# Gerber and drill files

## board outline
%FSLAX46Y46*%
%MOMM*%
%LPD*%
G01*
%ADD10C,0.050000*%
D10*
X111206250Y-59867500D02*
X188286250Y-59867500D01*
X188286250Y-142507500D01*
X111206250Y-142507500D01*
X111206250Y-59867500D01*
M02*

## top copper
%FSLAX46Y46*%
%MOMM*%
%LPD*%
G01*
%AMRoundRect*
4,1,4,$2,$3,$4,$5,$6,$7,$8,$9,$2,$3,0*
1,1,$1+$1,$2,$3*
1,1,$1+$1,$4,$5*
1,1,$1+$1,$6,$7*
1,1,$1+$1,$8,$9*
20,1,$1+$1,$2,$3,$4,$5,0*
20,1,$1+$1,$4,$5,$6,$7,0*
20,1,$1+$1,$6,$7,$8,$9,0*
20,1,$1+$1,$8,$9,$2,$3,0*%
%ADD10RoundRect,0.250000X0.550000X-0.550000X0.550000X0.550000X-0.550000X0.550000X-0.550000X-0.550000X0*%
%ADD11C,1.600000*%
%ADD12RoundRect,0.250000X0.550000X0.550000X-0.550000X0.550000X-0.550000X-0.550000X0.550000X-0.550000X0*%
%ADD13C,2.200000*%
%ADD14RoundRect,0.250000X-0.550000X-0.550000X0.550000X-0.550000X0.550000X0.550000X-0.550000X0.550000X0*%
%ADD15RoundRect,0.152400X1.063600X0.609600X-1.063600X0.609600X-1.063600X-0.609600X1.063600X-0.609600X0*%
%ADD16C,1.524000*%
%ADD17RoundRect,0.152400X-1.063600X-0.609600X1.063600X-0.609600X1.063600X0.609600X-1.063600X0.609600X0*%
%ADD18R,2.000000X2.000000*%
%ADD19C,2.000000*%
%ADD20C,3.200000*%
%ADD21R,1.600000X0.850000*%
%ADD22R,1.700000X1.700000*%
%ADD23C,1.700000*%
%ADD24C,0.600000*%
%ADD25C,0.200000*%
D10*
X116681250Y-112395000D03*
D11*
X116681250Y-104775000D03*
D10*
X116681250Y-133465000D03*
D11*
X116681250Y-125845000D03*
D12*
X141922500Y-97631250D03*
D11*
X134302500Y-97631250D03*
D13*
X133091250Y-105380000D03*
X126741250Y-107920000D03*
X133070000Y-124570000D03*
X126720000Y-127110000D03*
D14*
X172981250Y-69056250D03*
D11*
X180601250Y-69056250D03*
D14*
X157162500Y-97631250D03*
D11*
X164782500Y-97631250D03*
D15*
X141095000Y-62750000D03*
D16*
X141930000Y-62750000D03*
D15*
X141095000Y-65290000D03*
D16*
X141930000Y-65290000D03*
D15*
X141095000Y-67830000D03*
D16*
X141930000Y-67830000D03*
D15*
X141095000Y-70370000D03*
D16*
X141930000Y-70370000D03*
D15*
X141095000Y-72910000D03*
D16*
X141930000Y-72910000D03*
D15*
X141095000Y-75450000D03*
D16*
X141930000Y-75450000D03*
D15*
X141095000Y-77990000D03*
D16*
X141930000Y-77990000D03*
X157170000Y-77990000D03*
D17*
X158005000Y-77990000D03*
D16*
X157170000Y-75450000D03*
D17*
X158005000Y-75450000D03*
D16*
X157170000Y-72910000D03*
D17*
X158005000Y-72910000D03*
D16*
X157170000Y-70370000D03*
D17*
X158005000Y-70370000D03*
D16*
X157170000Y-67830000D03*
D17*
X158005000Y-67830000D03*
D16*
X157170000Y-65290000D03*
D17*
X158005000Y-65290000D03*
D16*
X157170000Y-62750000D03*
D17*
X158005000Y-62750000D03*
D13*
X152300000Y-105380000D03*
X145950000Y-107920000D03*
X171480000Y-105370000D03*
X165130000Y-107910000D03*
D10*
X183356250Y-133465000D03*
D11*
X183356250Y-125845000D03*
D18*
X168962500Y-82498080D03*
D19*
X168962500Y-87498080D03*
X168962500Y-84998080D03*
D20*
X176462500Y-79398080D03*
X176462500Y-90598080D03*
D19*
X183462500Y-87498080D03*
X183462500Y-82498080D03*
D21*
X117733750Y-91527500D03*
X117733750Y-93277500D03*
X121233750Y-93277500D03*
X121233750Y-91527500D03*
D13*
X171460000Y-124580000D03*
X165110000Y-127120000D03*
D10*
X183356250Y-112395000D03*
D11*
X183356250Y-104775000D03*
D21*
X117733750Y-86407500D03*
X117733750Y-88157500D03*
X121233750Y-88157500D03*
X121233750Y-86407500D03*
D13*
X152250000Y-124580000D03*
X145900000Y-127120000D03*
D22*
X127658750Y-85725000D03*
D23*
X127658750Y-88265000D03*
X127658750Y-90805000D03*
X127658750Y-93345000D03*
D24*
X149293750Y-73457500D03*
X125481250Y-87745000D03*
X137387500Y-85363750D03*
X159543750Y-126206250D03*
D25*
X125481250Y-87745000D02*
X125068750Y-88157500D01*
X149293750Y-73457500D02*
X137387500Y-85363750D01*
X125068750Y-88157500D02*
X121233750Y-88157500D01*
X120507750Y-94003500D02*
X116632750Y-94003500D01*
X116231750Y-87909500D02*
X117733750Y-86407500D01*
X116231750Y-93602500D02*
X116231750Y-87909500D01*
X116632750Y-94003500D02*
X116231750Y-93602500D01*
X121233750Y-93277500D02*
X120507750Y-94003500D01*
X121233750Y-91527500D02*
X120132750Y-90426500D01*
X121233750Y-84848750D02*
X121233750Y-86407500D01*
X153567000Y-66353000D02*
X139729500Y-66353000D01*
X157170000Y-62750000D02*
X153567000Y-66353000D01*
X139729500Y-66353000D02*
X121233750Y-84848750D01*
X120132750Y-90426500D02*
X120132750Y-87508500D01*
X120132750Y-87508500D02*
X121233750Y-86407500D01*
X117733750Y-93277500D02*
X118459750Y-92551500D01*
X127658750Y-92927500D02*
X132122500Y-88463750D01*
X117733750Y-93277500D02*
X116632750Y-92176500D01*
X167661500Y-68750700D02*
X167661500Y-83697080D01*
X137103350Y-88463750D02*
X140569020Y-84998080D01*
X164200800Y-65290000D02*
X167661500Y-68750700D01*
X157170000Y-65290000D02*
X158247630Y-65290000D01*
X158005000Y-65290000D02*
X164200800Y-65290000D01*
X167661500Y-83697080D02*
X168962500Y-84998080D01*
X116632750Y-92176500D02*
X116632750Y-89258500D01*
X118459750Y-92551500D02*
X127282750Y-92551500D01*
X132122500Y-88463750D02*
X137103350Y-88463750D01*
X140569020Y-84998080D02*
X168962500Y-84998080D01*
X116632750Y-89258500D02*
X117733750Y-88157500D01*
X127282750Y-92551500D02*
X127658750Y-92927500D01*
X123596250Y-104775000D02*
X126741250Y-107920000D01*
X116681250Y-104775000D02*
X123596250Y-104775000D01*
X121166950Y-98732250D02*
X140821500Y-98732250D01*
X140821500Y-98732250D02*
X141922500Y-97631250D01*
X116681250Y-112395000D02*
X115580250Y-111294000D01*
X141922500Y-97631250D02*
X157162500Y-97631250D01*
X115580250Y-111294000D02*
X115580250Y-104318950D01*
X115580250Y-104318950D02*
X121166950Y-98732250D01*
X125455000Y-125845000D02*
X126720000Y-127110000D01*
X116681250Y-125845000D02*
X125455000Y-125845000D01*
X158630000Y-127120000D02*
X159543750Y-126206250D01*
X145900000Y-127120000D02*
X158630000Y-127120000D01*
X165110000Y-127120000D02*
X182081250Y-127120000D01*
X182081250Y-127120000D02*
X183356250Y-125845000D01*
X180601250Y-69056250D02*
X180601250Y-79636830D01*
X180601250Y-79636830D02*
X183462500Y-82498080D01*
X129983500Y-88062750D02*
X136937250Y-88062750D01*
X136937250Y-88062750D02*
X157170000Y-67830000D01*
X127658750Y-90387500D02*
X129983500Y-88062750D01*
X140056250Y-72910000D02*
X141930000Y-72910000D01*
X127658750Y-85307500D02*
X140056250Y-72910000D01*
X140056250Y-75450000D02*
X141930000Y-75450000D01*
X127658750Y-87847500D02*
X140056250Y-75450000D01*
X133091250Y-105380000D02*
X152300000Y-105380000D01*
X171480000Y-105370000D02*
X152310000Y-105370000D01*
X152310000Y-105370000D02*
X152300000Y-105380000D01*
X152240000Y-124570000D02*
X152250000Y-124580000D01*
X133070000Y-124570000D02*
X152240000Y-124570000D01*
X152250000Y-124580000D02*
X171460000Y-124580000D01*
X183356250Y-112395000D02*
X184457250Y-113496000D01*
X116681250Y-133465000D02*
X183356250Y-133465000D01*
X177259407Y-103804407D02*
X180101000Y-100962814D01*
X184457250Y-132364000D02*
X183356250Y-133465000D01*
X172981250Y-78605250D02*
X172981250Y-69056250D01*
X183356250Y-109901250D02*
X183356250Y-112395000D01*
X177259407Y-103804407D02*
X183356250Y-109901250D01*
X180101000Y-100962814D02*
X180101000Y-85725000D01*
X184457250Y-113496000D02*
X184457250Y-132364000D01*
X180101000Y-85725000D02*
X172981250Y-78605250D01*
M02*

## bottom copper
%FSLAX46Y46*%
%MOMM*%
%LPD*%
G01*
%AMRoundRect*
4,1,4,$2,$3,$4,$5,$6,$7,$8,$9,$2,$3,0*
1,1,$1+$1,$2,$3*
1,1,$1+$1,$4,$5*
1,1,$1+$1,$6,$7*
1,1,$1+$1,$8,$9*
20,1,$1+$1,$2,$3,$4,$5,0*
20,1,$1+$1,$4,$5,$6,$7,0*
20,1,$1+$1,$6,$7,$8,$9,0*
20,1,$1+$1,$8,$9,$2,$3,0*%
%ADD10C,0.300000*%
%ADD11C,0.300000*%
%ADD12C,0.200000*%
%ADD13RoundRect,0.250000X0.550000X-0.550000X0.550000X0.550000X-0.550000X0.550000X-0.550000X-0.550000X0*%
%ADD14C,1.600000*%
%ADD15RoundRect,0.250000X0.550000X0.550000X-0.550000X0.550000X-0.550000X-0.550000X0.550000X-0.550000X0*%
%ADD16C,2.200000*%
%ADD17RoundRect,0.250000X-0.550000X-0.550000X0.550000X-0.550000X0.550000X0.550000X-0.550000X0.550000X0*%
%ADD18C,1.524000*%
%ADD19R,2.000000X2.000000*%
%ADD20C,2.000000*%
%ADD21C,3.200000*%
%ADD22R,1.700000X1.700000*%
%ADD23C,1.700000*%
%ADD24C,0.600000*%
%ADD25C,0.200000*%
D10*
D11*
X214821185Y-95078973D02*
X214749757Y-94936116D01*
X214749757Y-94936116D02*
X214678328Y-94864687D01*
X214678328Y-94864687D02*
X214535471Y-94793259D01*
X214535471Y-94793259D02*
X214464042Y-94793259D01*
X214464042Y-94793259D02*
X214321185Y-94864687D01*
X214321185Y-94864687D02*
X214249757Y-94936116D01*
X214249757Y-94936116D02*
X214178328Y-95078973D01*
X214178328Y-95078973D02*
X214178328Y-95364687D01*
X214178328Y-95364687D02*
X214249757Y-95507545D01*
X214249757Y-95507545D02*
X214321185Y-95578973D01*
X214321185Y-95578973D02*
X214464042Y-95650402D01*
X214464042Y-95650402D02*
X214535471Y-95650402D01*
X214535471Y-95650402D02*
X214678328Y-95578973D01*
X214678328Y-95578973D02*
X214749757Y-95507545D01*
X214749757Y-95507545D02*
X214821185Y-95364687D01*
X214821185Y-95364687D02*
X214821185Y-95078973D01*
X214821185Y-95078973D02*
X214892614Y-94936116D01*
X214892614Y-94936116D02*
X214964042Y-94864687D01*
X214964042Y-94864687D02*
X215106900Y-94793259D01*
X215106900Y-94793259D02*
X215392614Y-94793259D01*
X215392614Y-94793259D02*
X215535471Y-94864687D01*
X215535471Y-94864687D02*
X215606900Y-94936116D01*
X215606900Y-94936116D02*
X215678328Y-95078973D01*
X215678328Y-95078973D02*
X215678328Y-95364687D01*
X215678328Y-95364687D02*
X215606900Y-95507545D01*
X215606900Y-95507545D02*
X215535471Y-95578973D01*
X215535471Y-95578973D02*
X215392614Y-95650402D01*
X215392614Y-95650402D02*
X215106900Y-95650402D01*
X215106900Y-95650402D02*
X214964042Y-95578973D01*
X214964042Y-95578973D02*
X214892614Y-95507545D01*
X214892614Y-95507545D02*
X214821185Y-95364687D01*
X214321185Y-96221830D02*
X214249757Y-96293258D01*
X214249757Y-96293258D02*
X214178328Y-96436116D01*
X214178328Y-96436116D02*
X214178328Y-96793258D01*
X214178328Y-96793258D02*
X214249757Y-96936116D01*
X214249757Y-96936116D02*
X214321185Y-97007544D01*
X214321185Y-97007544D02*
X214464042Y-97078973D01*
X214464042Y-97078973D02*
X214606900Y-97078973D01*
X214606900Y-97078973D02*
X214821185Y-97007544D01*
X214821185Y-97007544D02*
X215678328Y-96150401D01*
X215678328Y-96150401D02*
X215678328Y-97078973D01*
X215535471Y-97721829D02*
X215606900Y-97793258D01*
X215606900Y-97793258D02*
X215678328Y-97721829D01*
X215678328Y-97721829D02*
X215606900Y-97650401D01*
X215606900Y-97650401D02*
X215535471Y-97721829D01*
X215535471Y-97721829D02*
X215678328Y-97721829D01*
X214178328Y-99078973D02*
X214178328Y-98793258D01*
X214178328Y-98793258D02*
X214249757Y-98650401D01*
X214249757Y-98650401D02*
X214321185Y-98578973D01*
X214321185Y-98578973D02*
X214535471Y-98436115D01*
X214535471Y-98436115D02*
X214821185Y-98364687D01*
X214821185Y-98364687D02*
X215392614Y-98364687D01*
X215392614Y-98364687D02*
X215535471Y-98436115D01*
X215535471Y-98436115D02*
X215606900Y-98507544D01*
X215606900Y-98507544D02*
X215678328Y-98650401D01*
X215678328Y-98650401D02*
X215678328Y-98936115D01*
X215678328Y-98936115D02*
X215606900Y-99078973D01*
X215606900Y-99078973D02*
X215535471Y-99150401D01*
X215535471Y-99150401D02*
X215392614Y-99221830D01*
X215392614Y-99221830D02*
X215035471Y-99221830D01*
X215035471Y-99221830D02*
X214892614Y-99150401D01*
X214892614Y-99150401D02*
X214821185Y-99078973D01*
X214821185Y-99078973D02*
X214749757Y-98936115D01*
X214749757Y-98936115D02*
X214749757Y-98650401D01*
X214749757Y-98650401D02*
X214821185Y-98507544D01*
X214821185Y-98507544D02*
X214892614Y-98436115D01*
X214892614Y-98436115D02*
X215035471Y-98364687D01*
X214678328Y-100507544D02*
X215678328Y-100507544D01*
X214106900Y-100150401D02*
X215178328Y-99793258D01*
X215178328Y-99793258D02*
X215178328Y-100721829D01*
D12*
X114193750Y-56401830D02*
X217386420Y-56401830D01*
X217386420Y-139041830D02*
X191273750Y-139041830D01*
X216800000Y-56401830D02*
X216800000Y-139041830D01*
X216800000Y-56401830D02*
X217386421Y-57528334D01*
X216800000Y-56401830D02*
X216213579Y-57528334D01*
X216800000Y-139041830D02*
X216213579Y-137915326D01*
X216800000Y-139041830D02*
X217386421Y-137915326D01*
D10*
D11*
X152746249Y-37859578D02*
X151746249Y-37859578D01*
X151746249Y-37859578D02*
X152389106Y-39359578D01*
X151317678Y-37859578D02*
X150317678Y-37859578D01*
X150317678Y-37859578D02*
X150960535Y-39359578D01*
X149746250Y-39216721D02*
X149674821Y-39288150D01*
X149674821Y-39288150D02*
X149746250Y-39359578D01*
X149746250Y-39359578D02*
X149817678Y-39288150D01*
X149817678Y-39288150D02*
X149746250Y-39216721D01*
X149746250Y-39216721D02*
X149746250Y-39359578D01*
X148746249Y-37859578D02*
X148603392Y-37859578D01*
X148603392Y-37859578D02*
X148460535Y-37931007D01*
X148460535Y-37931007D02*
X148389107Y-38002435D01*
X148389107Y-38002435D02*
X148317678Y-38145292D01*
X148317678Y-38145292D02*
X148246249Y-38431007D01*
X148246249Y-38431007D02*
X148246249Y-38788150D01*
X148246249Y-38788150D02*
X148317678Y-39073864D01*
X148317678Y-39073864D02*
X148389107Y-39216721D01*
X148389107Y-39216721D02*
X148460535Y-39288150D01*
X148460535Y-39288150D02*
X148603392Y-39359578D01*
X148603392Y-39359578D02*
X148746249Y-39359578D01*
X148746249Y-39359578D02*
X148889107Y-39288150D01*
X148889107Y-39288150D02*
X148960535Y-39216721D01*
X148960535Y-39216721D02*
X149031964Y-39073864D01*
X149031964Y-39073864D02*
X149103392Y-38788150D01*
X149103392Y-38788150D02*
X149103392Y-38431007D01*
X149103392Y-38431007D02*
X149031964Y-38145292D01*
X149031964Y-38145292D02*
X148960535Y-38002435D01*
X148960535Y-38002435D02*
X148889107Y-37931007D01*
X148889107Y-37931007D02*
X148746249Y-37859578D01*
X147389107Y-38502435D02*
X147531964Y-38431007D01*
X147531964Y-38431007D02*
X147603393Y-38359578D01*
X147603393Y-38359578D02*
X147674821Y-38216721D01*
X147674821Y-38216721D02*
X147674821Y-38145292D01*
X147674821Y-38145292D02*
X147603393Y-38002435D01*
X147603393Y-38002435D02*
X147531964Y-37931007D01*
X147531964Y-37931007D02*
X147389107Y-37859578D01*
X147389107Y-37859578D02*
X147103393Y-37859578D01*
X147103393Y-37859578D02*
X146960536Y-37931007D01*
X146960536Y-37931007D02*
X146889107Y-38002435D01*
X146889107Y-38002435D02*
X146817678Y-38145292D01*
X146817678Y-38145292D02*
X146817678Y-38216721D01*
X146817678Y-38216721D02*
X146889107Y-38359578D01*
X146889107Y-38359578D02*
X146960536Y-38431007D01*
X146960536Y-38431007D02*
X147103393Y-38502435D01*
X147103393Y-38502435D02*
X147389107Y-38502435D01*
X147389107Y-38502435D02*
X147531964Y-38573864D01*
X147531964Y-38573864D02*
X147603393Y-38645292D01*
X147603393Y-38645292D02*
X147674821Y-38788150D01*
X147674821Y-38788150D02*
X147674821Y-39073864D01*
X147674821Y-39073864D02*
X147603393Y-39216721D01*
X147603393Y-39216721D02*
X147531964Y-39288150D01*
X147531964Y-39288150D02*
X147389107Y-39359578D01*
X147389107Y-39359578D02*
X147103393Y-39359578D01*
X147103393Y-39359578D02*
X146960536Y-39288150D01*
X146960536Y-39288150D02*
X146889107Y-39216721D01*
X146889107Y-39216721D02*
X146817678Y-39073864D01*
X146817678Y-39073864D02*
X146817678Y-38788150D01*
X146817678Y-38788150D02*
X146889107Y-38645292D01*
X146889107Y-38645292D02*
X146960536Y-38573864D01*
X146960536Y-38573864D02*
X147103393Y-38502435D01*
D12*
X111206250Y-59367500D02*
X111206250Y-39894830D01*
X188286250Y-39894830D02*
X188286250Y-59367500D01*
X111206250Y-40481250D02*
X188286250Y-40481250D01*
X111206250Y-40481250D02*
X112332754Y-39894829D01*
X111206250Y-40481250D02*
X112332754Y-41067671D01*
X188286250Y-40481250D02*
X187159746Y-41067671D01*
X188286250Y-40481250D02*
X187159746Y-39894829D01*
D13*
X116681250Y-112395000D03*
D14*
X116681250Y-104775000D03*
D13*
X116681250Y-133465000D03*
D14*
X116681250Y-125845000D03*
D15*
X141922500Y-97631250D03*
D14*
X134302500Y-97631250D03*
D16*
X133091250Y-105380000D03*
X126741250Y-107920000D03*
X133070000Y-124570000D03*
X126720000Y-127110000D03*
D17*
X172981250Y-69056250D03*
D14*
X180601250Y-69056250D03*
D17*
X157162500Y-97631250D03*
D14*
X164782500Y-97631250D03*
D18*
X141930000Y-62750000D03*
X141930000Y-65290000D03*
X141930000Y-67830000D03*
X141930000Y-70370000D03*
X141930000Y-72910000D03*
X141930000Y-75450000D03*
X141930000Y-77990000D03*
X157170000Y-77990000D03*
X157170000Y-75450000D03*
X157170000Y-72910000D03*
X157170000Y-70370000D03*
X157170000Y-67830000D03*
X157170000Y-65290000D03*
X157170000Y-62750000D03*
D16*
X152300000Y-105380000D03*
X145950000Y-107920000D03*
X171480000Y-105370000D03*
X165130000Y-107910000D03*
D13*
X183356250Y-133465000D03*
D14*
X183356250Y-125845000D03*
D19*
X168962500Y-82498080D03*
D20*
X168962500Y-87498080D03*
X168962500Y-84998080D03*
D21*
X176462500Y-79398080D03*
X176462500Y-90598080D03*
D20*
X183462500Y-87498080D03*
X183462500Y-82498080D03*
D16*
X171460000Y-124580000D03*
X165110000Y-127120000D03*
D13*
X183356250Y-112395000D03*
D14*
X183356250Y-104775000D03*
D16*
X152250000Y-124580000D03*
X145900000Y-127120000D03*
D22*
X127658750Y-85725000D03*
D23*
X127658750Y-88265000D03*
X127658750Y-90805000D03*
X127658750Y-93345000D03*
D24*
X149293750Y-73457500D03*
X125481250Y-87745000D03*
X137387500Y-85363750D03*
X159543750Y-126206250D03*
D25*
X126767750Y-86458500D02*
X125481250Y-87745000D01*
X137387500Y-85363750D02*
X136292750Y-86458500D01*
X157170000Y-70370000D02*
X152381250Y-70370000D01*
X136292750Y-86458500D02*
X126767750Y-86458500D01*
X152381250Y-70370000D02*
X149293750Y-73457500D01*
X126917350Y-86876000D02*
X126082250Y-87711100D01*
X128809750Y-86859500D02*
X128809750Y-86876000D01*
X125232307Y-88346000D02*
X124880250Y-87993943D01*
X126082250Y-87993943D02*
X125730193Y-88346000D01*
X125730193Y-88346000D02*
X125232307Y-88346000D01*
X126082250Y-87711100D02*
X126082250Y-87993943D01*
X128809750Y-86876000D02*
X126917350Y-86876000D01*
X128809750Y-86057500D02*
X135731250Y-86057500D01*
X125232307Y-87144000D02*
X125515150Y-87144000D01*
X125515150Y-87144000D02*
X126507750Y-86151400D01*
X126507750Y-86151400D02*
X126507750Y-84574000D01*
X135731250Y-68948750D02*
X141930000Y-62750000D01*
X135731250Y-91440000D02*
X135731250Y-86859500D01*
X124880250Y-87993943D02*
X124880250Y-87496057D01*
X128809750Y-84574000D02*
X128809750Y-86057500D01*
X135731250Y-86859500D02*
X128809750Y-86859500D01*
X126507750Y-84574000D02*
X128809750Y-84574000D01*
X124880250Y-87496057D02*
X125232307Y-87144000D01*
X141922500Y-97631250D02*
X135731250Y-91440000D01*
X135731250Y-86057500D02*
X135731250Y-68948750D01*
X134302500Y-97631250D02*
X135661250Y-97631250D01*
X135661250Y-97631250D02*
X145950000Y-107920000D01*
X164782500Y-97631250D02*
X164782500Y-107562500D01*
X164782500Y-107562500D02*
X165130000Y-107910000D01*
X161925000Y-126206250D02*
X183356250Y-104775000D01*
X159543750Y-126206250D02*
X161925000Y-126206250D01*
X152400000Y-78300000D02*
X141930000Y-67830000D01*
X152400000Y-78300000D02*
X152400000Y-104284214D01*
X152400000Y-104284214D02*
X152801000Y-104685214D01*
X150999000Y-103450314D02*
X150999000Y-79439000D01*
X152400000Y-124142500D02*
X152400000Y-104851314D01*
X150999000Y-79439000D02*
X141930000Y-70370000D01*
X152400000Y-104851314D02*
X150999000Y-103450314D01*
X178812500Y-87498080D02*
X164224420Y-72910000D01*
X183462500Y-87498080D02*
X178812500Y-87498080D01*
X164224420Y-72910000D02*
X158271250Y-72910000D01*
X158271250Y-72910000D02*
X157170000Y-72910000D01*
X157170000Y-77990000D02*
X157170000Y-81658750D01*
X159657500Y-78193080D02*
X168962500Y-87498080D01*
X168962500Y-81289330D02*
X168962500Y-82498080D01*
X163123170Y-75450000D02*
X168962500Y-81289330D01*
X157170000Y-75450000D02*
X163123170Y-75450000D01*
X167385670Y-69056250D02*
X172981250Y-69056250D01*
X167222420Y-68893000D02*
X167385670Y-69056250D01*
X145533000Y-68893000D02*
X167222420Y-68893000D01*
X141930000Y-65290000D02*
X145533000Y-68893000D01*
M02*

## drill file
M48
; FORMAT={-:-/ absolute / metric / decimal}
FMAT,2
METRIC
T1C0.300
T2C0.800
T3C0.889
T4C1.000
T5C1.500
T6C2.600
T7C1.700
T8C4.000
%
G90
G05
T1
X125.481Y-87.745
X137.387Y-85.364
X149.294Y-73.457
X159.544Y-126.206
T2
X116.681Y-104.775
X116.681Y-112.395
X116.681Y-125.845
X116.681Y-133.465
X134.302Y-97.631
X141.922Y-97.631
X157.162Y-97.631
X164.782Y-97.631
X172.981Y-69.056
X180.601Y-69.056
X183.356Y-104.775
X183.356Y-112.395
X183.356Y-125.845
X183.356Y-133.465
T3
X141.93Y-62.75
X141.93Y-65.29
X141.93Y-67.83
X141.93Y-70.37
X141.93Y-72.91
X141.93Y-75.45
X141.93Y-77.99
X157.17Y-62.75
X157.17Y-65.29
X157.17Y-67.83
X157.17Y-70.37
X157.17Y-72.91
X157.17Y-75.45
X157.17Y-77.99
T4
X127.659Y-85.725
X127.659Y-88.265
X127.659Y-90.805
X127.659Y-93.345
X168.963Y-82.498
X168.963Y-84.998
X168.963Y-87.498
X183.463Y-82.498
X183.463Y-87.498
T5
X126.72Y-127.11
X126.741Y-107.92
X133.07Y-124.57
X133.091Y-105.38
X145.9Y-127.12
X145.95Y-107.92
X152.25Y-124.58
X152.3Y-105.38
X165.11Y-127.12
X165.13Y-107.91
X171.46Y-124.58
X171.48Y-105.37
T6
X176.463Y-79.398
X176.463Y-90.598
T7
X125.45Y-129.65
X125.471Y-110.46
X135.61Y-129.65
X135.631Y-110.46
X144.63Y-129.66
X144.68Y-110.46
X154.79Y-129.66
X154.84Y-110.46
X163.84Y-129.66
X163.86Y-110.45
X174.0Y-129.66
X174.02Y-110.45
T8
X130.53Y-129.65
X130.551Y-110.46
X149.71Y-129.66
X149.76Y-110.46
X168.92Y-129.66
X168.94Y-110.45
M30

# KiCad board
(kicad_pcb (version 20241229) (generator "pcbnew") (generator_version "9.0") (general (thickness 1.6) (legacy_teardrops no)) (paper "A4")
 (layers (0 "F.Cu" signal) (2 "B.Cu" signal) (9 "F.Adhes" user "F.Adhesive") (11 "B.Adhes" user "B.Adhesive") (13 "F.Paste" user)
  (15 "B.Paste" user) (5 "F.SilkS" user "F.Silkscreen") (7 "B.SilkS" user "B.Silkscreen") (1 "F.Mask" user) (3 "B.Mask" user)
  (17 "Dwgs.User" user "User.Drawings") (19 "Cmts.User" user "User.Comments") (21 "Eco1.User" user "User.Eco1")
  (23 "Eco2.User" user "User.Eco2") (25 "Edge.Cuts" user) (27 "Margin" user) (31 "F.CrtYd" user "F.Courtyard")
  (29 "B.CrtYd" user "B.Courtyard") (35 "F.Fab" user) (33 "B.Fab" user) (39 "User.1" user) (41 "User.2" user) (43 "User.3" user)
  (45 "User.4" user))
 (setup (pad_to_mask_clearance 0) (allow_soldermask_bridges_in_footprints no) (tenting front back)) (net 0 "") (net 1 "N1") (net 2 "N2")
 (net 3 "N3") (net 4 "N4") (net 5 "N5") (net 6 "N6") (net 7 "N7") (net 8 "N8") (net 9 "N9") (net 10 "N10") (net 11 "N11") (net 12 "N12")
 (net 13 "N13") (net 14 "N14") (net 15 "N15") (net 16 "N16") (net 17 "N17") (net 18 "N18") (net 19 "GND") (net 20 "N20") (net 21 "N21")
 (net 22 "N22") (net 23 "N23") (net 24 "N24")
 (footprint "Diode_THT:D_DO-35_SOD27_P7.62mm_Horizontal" (layer "F.Cu") (at 116.68125 112.395 90)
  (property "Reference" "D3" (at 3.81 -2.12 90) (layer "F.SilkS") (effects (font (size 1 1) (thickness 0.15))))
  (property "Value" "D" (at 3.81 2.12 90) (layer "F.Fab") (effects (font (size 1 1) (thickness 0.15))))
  (pad "1" thru_hole roundrect (at 0 0 90) (size 1.6 1.6) (drill 0.8) (layers "*.Cu" "*.Mask") (remove_unused_layers no)
   (roundrect_rratio 0.15625) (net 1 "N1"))
  (pad "2" thru_hole circle (at 7.62 0 90) (size 1.6 1.6) (drill 0.8) (layers "*.Cu" "*.Mask") (remove_unused_layers no) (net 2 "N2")))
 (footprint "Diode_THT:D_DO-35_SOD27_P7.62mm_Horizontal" (layer "F.Cu") (at 116.68125 133.465 90)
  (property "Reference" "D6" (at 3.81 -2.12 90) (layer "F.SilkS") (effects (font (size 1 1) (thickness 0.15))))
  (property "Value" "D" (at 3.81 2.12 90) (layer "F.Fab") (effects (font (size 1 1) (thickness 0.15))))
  (pad "1" thru_hole roundrect (at 0 0 90) (size 1.6 1.6) (drill 0.8) (layers "*.Cu" "*.Mask") (remove_unused_layers no)
   (roundrect_rratio 0.15625) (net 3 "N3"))
  (pad "2" thru_hole circle (at 7.62 0 90) (size 1.6 1.6) (drill 0.8) (layers "*.Cu" "*.Mask") (remove_unused_layers no) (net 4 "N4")))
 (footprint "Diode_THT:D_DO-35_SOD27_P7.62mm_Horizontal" (layer "F.Cu") (at 141.9225 97.63125 180)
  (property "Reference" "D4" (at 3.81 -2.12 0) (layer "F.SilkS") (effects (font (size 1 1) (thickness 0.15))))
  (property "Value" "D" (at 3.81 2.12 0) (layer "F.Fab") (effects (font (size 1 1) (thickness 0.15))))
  (pad "1" thru_hole roundrect (at 0 0 180) (size 1.6 1.6) (drill 0.8) (layers "*.Cu" "*.Mask") (remove_unused_layers no)
   (roundrect_rratio 0.15625) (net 1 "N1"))
  (pad "2" thru_hole circle (at 7.62 0 180) (size 1.6 1.6) (drill 0.8) (layers "*.Cu" "*.Mask") (remove_unused_layers no) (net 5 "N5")))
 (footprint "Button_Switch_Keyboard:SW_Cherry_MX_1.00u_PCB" (layer "F.Cu") (at 133.09125 105.38)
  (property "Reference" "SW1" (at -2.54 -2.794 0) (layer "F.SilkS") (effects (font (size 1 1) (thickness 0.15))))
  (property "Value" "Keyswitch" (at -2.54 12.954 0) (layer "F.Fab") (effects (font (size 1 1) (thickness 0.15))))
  (pad "" np_thru_hole circle (at -7.62 5.08) (size 1.7 1.7) (drill 1.7) (layers "*.Cu" "*.Mask"))
  (pad "" np_thru_hole circle (at -2.54 5.08) (size 4 4) (drill 4) (layers "*.Cu" "*.Mask"))
  (pad "" np_thru_hole circle (at 2.54 5.08) (size 1.7 1.7) (drill 1.7) (layers "*.Cu" "*.Mask"))
  (pad "1" thru_hole circle (at 0 0) (size 2.2 2.2) (drill 1.5) (layers "*.Cu" "*.Mask") (remove_unused_layers no) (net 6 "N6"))
  (pad "2" thru_hole circle (at -6.35 2.54) (size 2.2 2.2) (drill 1.5) (layers "*.Cu" "*.Mask") (remove_unused_layers no) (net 2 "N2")))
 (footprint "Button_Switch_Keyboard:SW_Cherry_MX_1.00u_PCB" (layer "F.Cu") (at 133.07 124.57)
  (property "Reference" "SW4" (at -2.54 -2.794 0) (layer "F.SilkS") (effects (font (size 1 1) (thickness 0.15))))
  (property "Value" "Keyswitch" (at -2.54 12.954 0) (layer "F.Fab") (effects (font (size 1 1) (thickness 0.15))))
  (pad "" np_thru_hole circle (at -7.62 5.08) (size 1.7 1.7) (drill 1.7) (layers "*.Cu" "*.Mask"))
  (pad "" np_thru_hole circle (at -2.54 5.08) (size 4 4) (drill 4) (layers "*.Cu" "*.Mask"))
  (pad "" np_thru_hole circle (at 2.54 5.08) (size 1.7 1.7) (drill 1.7) (layers "*.Cu" "*.Mask"))
  (pad "1" thru_hole circle (at 0 0) (size 2.2 2.2) (drill 1.5) (layers "*.Cu" "*.Mask") (remove_unused_layers no) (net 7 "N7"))
  (pad "2" thru_hole circle (at -6.35 2.54) (size 2.2 2.2) (drill 1.5) (layers "*.Cu" "*.Mask") (remove_unused_layers no) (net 4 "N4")))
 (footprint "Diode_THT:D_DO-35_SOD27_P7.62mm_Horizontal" (layer "F.Cu") (at 172.98125 69.05625)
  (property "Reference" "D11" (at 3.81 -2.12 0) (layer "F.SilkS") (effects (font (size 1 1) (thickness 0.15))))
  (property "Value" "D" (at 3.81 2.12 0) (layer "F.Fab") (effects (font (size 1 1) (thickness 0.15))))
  (pad "1" thru_hole roundrect (at 0 0) (size 1.6 1.6) (drill 0.8) (layers "*.Cu" "*.Mask") (remove_unused_layers no)
   (roundrect_rratio 0.15625) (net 3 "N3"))
  (pad "2" thru_hole circle (at 7.62 0) (size 1.6 1.6) (drill 0.8) (layers "*.Cu" "*.Mask") (remove_unused_layers no) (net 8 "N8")))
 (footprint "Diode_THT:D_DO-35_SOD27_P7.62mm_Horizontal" (layer "F.Cu") (at 157.1625 97.63125)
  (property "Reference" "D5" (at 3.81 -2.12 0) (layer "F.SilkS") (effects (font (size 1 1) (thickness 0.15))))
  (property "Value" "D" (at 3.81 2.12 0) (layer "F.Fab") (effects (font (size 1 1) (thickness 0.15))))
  (pad "1" thru_hole roundrect (at 0 0) (size 1.6 1.6) (drill 0.8) (layers "*.Cu" "*.Mask") (remove_unused_layers no)
   (roundrect_rratio 0.15625) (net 1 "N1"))
  (pad "2" thru_hole circle (at 7.62 0) (size 1.6 1.6) (drill 0.8) (layers "*.Cu" "*.Mask") (remove_unused_layers no) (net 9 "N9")))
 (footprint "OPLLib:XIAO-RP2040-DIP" (layer "F.Cu") (at 149.55 70.37)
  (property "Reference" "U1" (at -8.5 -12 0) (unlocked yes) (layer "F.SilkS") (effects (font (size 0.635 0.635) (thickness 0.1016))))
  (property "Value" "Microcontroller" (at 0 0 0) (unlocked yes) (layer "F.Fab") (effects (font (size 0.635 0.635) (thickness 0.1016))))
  (pad "1" smd roundrect (at -8.455 -7.62 180) (size 2.432 1.524) (layers "F.Cu" "F.Mask") (roundrect_rratio 0.1) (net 1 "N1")
   (thermal_bridge_angle 45))
  (pad "1" thru_hole circle (at -7.62 -7.62 180) (size 1.524 1.524) (drill 0.889) (layers "*.Cu" "*.Mask") (remove_unused_layers no)
   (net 1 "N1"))
  (pad "2" smd roundrect (at -8.455 -5.08 180) (size 2.432 1.524) (layers "F.Cu" "F.Mask") (roundrect_rratio 0.1) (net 3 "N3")
   (thermal_bridge_angle 45))
  (pad "2" thru_hole circle (at -7.62 -5.08 180) (size 1.524 1.524) (drill 0.889) (layers "*.Cu" "*.Mask") (remove_unused_layers no)
   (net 3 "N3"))
  (pad "3" smd roundrect (at -8.455 -2.54 180) (size 2.432 1.524) (layers "F.Cu" "F.Mask") (roundrect_rratio 0.1) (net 6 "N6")
   (thermal_bridge_angle 45))
  (pad "3" thru_hole circle (at -7.62 -2.54 180) (size 1.524 1.524) (drill 0.889) (layers "*.Cu" "*.Mask") (remove_unused_layers no)
   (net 6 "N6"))
  (pad "4" smd roundrect (at -8.455 0 180) (size 2.432 1.524) (layers "F.Cu" "F.Mask") (roundrect_rratio 0.1) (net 7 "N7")
   (thermal_bridge_angle 45))
  (pad "4" thru_hole circle (at -7.62 0 180) (size 1.524 1.524) (drill 0.889) (layers "*.Cu" "*.Mask") (remove_unused_layers no)
   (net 7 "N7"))
  (pad "5" smd roundrect (at -8.455 2.54 180) (size 2.432 1.524) (layers "F.Cu" "F.Mask") (roundrect_rratio 0.1) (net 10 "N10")
   (thermal_bridge_angle 45))
  (pad "5" thru_hole circle (at -7.62 2.54 180) (size 1.524 1.524) (drill 0.889) (layers "*.Cu" "*.Mask") (remove_unused_layers no)
   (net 10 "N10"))
  (pad "6" smd roundrect (at -8.455 5.08 180) (size 2.432 1.524) (layers "F.Cu" "F.Mask") (roundrect_rratio 0.1) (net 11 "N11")
   (thermal_bridge_angle 45))
  (pad "6" thru_hole circle (at -7.62 5.08 180) (size 1.524 1.524) (drill 0.889) (layers "*.Cu" "*.Mask") (remove_unused_layers no)
   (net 11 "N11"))
  (pad "7" smd roundrect (at -8.455 7.62 180) (size 2.432 1.524) (layers "F.Cu" "F.Mask") (roundrect_rratio 0.1) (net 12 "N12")
   (thermal_bridge_angle 45))
  (pad "7" thru_hole circle (at -7.62 7.62 180) (size 1.524 1.524) (drill 0.889) (layers "*.Cu" "*.Mask") (remove_unused_layers no)
   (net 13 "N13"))
  (pad "8" thru_hole circle (at 7.62 7.62) (size 1.524 1.524) (drill 0.889) (layers "*.Cu" "*.Mask") (remove_unused_layers no)
   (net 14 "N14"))
  (pad "8" smd roundrect (at 8.455 7.62) (size 2.432 1.524) (layers "F.Cu" "F.Mask") (roundrect_rratio 0.1) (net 14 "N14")
   (thermal_bridge_angle 45))
  (pad "9" thru_hole circle (at 7.62 5.08) (size 1.524 1.524) (drill 0.889) (layers "*.Cu" "*.Mask") (remove_unused_layers no)
   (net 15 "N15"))
  (pad "9" smd roundrect (at 8.455 5.08) (size 2.432 1.524) (layers "F.Cu" "F.Mask") (roundrect_rratio 0.1) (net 15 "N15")
   (thermal_bridge_angle 45))
  (pad "10" thru_hole circle (at 7.62 2.54) (size 1.524 1.524) (drill 0.889) (layers "*.Cu" "*.Mask") (remove_unused_layers no)
   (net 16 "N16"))
  (pad "10" smd roundrect (at 8.455 2.54) (size 2.432 1.524) (layers "F.Cu" "F.Mask") (roundrect_rratio 0.1) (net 16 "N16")
   (thermal_bridge_angle 45))
  (pad "11" thru_hole circle (at 7.62 0) (size 1.524 1.524) (drill 0.889) (layers "*.Cu" "*.Mask") (remove_unused_layers no) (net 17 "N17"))
  (pad "11" smd roundrect (at 8.455 0) (size 2.432 1.524) (layers "F.Cu" "F.Mask") (roundrect_rratio 0.1) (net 17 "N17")
   (thermal_bridge_angle 45))
  (pad "12" thru_hole circle (at 7.62 -2.54) (size 1.524 1.524) (drill 0.889) (layers "*.Cu" "*.Mask") (remove_unused_layers no)
   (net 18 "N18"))
  (pad "12" smd roundrect (at 8.455 -2.54) (size 2.432 1.524) (layers "F.Cu" "F.Mask") (roundrect_rratio 0.1) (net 18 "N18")
   (thermal_bridge_angle 45))
  (pad "13" thru_hole circle (at 7.62 -5.08) (size 1.524 1.524) (drill 0.889) (layers "*.Cu" "*.Mask") (remove_unused_layers no)
   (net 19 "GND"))
  (pad "13" smd roundrect (at 8.455 -5.08) (size 2.432 1.524) (layers "F.Cu" "F.Mask") (roundrect_rratio 0.1) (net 19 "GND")
   (thermal_bridge_angle 45))
  (pad "14" thru_hole circle (at 7.62 -7.62) (size 1.524 1.524) (drill 0.889) (layers "*.Cu" "*.Mask") (remove_unused_layers no)
   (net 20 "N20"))
  (pad "14" smd roundrect (at 8.455 -7.62) (size 2.432 1.524) (layers "F.Cu" "F.Mask") (roundrect_rratio 0.1) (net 20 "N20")
   (thermal_bridge_angle 45)))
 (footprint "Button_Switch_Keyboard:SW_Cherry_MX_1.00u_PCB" (layer "F.Cu") (at 152.3 105.38)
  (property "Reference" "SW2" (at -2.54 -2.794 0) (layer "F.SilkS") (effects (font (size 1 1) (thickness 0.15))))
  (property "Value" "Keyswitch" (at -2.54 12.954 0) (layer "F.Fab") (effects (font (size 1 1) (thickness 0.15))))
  (pad "" np_thru_hole circle (at -7.62 5.08) (size 1.7 1.7) (drill 1.7) (layers "*.Cu" "*.Mask"))
  (pad "" np_thru_hole circle (at -2.54 5.08) (size 4 4) (drill 4) (layers "*.Cu" "*.Mask"))
  (pad "" np_thru_hole circle (at 2.54 5.08) (size 1.7 1.7) (drill 1.7) (layers "*.Cu" "*.Mask"))
  (pad "1" thru_hole circle (at 0 0) (size 2.2 2.2) (drill 1.5) (layers "*.Cu" "*.Mask") (remove_unused_layers no) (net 6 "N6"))
  (pad "2" thru_hole circle (at -6.35 2.54) (size 2.2 2.2) (drill 1.5) (layers "*.Cu" "*.Mask") (remove_unused_layers no) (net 5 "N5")))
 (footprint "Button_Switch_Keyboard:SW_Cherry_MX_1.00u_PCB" (layer "F.Cu") (at 171.48 105.37)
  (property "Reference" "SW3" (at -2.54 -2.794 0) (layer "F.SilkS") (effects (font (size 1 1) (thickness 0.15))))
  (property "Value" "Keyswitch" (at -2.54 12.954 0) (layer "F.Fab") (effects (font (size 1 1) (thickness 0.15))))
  (pad "" np_thru_hole circle (at -7.62 5.08) (size 1.7 1.7) (drill 1.7) (layers "*.Cu" "*.Mask"))
  (pad "" np_thru_hole circle (at -2.54 5.08) (size 4 4) (drill 4) (layers "*.Cu" "*.Mask"))
  (pad "" np_thru_hole circle (at 2.54 5.08) (size 1.7 1.7) (drill 1.7) (layers "*.Cu" "*.Mask"))
  (pad "1" thru_hole circle (at 0 0) (size 2.2 2.2) (drill 1.5) (layers "*.Cu" "*.Mask") (remove_unused_layers no) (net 6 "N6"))
  (pad "2" thru_hole circle (at -6.35 2.54) (size 2.2 2.2) (drill 1.5) (layers "*.Cu" "*.Mask") (remove_unused_layers no) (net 9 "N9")))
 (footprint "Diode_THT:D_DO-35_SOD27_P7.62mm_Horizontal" (layer "F.Cu") (at 183.35625 133.465 90)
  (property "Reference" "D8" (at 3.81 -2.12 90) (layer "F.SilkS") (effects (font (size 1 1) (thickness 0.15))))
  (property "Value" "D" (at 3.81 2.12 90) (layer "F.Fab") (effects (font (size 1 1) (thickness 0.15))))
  (pad "1" thru_hole roundrect (at 0 0 90) (size 1.6 1.6) (drill 0.8) (layers "*.Cu" "*.Mask") (remove_unused_layers no)
   (roundrect_rratio 0.15625) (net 3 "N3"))
  (pad "2" thru_hole circle (at 7.62 0 90) (size 1.6 1.6) (drill 0.8) (layers "*.Cu" "*.Mask") (remove_unused_layers no) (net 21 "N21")))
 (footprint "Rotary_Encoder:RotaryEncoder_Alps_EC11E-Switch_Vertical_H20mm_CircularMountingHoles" (layer "F.Cu") (at 168.9625 82.49808)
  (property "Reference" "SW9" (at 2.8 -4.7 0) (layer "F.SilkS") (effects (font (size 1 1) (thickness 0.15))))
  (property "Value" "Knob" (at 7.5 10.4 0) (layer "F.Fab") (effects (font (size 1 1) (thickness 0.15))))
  (pad "A" thru_hole rect (at 0 0) (size 2 2) (drill 1) (layers "*.Cu" "*.Mask") (remove_unused_layers no) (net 15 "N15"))
  (pad "B" thru_hole circle (at 0 5) (size 2 2) (drill 1) (layers "*.Cu" "*.Mask") (remove_unused_layers no) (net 14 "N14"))
  (pad "C" thru_hole circle (at 0 2.5) (size 2 2) (drill 1) (layers "*.Cu" "*.Mask") (remove_unused_layers no) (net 19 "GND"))
  (pad "MP" thru_hole circle (at 7.5 -3.1) (size 3.2 3.2) (drill 2.6) (layers "*.Cu" "*.Mask") (remove_unused_layers no))
  (pad "MP" thru_hole circle (at 7.5 8.1) (size 3.2 3.2) (drill 2.6) (layers "*.Cu" "*.Mask") (remove_unused_layers no))
  (pad "S1" thru_hole circle (at 14.5 5) (size 2 2) (drill 1) (layers "*.Cu" "*.Mask") (remove_unused_layers no) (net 16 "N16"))
  (pad "S2" thru_hole circle (at 14.5 0) (size 2 2) (drill 1) (layers "*.Cu" "*.Mask") (remove_unused_layers no) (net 8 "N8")))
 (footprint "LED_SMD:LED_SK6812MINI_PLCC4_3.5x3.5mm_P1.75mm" (layer "F.Cu") (at 119.48375 92.4025)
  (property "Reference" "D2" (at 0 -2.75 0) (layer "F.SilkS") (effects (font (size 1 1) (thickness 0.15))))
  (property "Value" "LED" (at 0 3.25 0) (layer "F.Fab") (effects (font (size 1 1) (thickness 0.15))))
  (pad "1" smd rect (at -1.75 -0.875) (size 1.6 0.85) (layers "F.Cu" "F.Mask" "F.Paste") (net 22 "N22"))
  (pad "2" smd rect (at -1.75 0.875) (size 1.6 0.85) (layers "F.Cu" "F.Mask" "F.Paste") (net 19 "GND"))
  (pad "3" smd rect (at 1.75 0.875) (size 1.6 0.85) (layers "F.Cu" "F.Mask" "F.Paste") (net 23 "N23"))
  (pad "4" smd rect (at 1.75 -0.875) (size 1.6 0.85) (layers "F.Cu" "F.Mask" "F.Paste") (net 20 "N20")))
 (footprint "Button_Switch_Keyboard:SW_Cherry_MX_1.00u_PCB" (layer "F.Cu") (at 171.46 124.58)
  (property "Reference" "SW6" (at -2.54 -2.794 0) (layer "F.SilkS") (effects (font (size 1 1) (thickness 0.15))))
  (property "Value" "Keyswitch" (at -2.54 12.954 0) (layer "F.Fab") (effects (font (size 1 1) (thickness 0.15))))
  (pad "" np_thru_hole circle (at -7.62 5.08) (size 1.7 1.7) (drill 1.7) (layers "*.Cu" "*.Mask"))
  (pad "" np_thru_hole circle (at -2.54 5.08) (size 4 4) (drill 4) (layers "*.Cu" "*.Mask"))
  (pad "" np_thru_hole circle (at 2.54 5.08) (size 1.7 1.7) (drill 1.7) (layers "*.Cu" "*.Mask"))
  (pad "1" thru_hole circle (at 0 0) (size 2.2 2.2) (drill 1.5) (layers "*.Cu" "*.Mask") (remove_unused_layers no) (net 7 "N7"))
  (pad "2" thru_hole circle (at -6.35 2.54) (size 2.2 2.2) (drill 1.5) (layers "*.Cu" "*.Mask") (remove_unused_layers no) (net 21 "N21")))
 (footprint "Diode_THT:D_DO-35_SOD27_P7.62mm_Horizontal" (layer "F.Cu") (at 183.35625 112.395 90)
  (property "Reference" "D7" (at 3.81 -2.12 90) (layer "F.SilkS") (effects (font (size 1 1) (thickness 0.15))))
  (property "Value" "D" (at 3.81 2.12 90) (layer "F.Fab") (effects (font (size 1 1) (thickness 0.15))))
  (pad "1" thru_hole roundrect (at 0 0 90) (size 1.6 1.6) (drill 0.8) (layers "*.Cu" "*.Mask") (remove_unused_layers no)
   (roundrect_rratio 0.15625) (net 3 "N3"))
  (pad "2" thru_hole circle (at 7.62 0 90) (size 1.6 1.6) (drill 0.8) (layers "*.Cu" "*.Mask") (remove_unused_layers no) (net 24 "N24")))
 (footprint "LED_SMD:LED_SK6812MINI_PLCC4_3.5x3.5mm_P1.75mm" (layer "F.Cu") (at 119.48375 87.2825)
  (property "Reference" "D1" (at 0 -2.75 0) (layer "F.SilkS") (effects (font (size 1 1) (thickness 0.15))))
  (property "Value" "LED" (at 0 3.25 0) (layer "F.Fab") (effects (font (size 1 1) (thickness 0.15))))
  (pad "1" smd rect (at -1.75 -0.875) (size 1.6 0.85) (layers "F.Cu" "F.Mask" "F.Paste") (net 23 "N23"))
  (pad "2" smd rect (at -1.75 0.875) (size 1.6 0.85) (layers "F.Cu" "F.Mask" "F.Paste") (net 19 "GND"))
  (pad "3" smd rect (at 1.75 0.875) (size 1.6 0.85) (layers "F.Cu" "F.Mask" "F.Paste") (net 17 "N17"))
  (pad "4" smd rect (at 1.75 -0.875) (size 1.6 0.85) (layers "F.Cu" "F.Mask" "F.Paste") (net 20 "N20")))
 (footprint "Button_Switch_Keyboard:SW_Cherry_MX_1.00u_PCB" (layer "F.Cu") (at 152.25 124.58)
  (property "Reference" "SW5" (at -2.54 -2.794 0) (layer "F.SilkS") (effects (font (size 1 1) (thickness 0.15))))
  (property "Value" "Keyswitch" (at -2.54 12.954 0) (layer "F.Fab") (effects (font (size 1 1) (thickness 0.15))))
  (pad "" np_thru_hole circle (at -7.62 5.08) (size 1.7 1.7) (drill 1.7) (layers "*.Cu" "*.Mask"))
  (pad "" np_thru_hole circle (at -2.54 5.08) (size 4 4) (drill 4) (layers "*.Cu" "*.Mask"))
  (pad "" np_thru_hole circle (at 2.54 5.08) (size 1.7 1.7) (drill 1.7) (layers "*.Cu" "*.Mask"))
  (pad "1" thru_hole circle (at 0 0) (size 2.2 2.2) (drill 1.5) (layers "*.Cu" "*.Mask") (remove_unused_layers no) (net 7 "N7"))
  (pad "2" thru_hole circle (at -6.35 2.54) (size 2.2 2.2) (drill 1.5) (layers "*.Cu" "*.Mask") (remove_unused_layers no) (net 24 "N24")))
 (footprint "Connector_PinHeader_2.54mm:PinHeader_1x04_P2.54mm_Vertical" (layer "F.Cu") (at 127.65875 85.725)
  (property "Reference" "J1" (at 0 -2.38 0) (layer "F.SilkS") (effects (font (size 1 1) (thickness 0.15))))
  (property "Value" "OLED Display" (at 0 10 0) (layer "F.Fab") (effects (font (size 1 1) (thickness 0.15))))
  (pad "1" thru_hole rect (at 0 0) (size 1.7 1.7) (drill 1) (layers "*.Cu" "*.Mask") (remove_unused_layers no) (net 10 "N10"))
  (pad "2" thru_hole circle (at 0 2.54) (size 1.7 1.7) (drill 1) (layers "*.Cu" "*.Mask") (remove_unused_layers no) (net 11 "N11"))
  (pad "3" thru_hole circle (at 0 5.08) (size 1.7 1.7) (drill 1) (layers "*.Cu" "*.Mask") (remove_unused_layers no) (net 18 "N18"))
  (pad "4" thru_hole circle (at 0 7.62) (size 1.7 1.7) (drill 1) (layers "*.Cu" "*.Mask") (remove_unused_layers no) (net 19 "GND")))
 (gr_rect (start 111.20625 59.8675) (end 188.28625 142.5075) (stroke (width 0.05) (type solid)) (fill no) (layer "Edge.Cuts"))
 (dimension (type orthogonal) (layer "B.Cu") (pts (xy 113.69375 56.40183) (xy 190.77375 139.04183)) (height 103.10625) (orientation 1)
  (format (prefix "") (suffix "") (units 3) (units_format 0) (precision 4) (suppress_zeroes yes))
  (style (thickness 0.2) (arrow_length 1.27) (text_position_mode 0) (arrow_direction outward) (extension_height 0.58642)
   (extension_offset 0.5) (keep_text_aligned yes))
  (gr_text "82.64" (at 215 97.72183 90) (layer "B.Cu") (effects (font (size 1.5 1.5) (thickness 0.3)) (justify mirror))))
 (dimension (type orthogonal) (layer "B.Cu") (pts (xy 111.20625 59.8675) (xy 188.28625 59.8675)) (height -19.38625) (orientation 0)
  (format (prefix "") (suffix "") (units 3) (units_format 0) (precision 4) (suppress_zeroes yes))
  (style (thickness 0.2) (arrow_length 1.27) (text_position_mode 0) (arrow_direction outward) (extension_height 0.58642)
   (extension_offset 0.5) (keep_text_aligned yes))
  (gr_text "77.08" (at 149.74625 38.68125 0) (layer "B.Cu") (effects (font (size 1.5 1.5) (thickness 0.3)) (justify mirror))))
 (segment (start 125.48125 87.745) (end 125.06875 88.1575) (width 0.2) (layer "F.Cu") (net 17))
 (segment (start 149.29375 73.4575) (end 137.3875 85.36375) (width 0.2) (layer "F.Cu") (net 17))
 (segment (start 125.06875 88.1575) (end 121.23375 88.1575) (width 0.2) (layer "F.Cu") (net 17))
 (via (at 149.29375 73.4575) (size 0.6) (drill 0.3) (layers "F.Cu" "B.Cu") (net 17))
 (via (at 125.48125 87.745) (size 0.6) (drill 0.3) (layers "F.Cu" "B.Cu") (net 17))
 (via (at 137.3875 85.36375) (size 0.6) (drill 0.3) (layers "F.Cu" "B.Cu") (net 17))
 (segment (start 126.76775 86.4585) (end 125.48125 87.745) (width 0.2) (layer "B.Cu") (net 17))
 (segment (start 137.3875 85.36375) (end 136.29275 86.4585) (width 0.2) (layer "B.Cu") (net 17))
 (segment (start 157.17 70.37) (end 152.38125 70.37) (width 0.2) (layer "B.Cu") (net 17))
 (segment (start 136.29275 86.4585) (end 126.76775 86.4585) (width 0.2) (layer "B.Cu") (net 17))
 (segment (start 152.38125 70.37) (end 149.29375 73.4575) (width 0.2) (layer "B.Cu") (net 17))
 (segment (start 120.50775 94.0035) (end 116.63275 94.0035) (width 0.2) (layer "F.Cu") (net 23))
 (segment (start 116.23175 87.9095) (end 117.73375 86.4075) (width 0.2) (layer "F.Cu") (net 23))
 (segment (start 116.23175 93.6025) (end 116.23175 87.9095) (width 0.2) (layer "F.Cu") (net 23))
 (segment (start 116.63275 94.0035) (end 116.23175 93.6025) (width 0.2) (layer "F.Cu") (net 23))
 (segment (start 121.23375 93.2775) (end 120.50775 94.0035) (width 0.2) (layer "F.Cu") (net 23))
 (segment (start 121.23375 91.5275) (end 120.13275 90.4265) (width 0.2) (layer "F.Cu") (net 20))
 (segment (start 121.23375 84.84875) (end 121.23375 86.4075) (width 0.2) (layer "F.Cu") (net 20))
 (segment (start 153.567 66.353) (end 139.7295 66.353) (width 0.2) (layer "F.Cu") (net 20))
 (segment (start 157.17 62.75) (end 153.567 66.353) (width 0.2) (layer "F.Cu") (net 20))
 (segment (start 139.7295 66.353) (end 121.23375 84.84875) (width 0.2) (layer "F.Cu") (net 20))
 (segment (start 120.13275 90.4265) (end 120.13275 87.5085) (width 0.2) (layer "F.Cu") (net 20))
 (segment (start 120.13275 87.5085) (end 121.23375 86.4075) (width 0.2) (layer "F.Cu") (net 20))
 (segment (start 117.73375 93.2775) (end 118.45975 92.5515) (width 0.2) (layer "F.Cu") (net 19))
 (segment (start 127.65875 92.9275) (end 132.1225 88.46375) (width 0.2) (layer "F.Cu") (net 19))
 (segment (start 117.73375 93.2775) (end 116.63275 92.1765) (width 0.2) (layer "F.Cu") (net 19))
 (segment (start 167.6615 68.7507) (end 167.6615 83.69708) (width 0.2) (layer "F.Cu") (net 19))
 (segment (start 137.10335 88.46375) (end 140.56902 84.99808) (width 0.2) (layer "F.Cu") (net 19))
 (segment (start 164.2008 65.29) (end 167.6615 68.7507) (width 0.2) (layer "F.Cu") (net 19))
 (segment (start 157.17 65.29) (end 158.24763 65.29) (width 0.2) (layer "F.Cu") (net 19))
 (segment (start 158.005 65.29) (end 164.2008 65.29) (width 0.2) (layer "F.Cu") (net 19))
 (segment (start 167.6615 83.69708) (end 168.9625 84.99808) (width 0.2) (layer "F.Cu") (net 19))
 (segment (start 116.63275 92.1765) (end 116.63275 89.2585) (width 0.2) (layer "F.Cu") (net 19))
 (segment (start 118.45975 92.5515) (end 127.28275 92.5515) (width 0.2) (layer "F.Cu") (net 19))
 (segment (start 132.1225 88.46375) (end 137.10335 88.46375) (width 0.2) (layer "F.Cu") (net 19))
 (segment (start 140.56902 84.99808) (end 168.9625 84.99808) (width 0.2) (layer "F.Cu") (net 19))
 (segment (start 116.63275 89.2585) (end 117.73375 88.1575) (width 0.2) (layer "F.Cu") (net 19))
 (segment (start 127.28275 92.5515) (end 127.65875 92.9275) (width 0.2) (layer "F.Cu") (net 19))
 (segment (start 123.59625 104.775) (end 126.74125 107.92) (width 0.2) (layer "F.Cu") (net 2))
 (segment (start 116.68125 104.775) (end 123.59625 104.775) (width 0.2) (layer "F.Cu") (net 2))
 (segment (start 121.16695 98.73225) (end 140.8215 98.73225) (width 0.2) (layer "F.Cu") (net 1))
 (segment (start 140.8215 98.73225) (end 141.9225 97.63125) (width 0.2) (layer "F.Cu") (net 1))
 (segment (start 116.68125 112.395) (end 115.58025 111.294) (width 0.2) (layer "F.Cu") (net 1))
 (segment (start 141.9225 97.63125) (end 157.1625 97.63125) (width 0.2) (layer "F.Cu") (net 1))
 (segment (start 115.58025 111.294) (end 115.58025 104.31895) (width 0.2) (layer "F.Cu") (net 1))
 (segment (start 115.58025 104.31895) (end 121.16695 98.73225) (width 0.2) (layer "F.Cu") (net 1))
 (segment (start 126.91735 86.876) (end 126.08225 87.7111) (width 0.2) (layer "B.Cu") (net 1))
 (segment (start 128.80975 86.8595) (end 128.80975 86.876) (width 0.2) (layer "B.Cu") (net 1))
 (segment (start 125.232307 88.346) (end 124.88025 87.993943) (width 0.2) (layer "B.Cu") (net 1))
 (segment (start 126.08225 87.993943) (end 125.730193 88.346) (width 0.2) (layer "B.Cu") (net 1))
 (segment (start 125.730193 88.346) (end 125.232307 88.346) (width 0.2) (layer "B.Cu") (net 1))
 (segment (start 126.08225 87.7111) (end 126.08225 87.993943) (width 0.2) (layer "B.Cu") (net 1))
 (segment (start 128.80975 86.876) (end 126.91735 86.876) (width 0.2) (layer "B.Cu") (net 1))
 (segment (start 128.80975 86.0575) (end 135.73125 86.0575) (width 0.2) (layer "B.Cu") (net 1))
 (segment (start 125.232307 87.144) (end 125.51515 87.144) (width 0.2) (layer "B.Cu") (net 1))
 (segment (start 125.51515 87.144) (end 126.50775 86.1514) (width 0.2) (layer "B.Cu") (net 1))
 (segment (start 126.50775 86.1514) (end 126.50775 84.574) (width 0.2) (layer "B.Cu") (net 1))
 (segment (start 135.73125 68.94875) (end 141.93 62.75) (width 0.2) (layer "B.Cu") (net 1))
 (segment (start 135.73125 91.44) (end 135.73125 86.8595) (width 0.2) (layer "B.Cu") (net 1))
 (segment (start 124.88025 87.993943) (end 124.88025 87.496057) (width 0.2) (layer "B.Cu") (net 1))
 (segment (start 128.80975 84.574) (end 128.80975 86.0575) (width 0.2) (layer "B.Cu") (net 1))
 (segment (start 135.73125 86.8595) (end 128.80975 86.8595) (width 0.2) (layer "B.Cu") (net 1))
 (segment (start 126.50775 84.574) (end 128.80975 84.574) (width 0.2) (layer "B.Cu") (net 1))
 (segment (start 124.88025 87.496057) (end 125.232307 87.144) (width 0.2) (layer "B.Cu") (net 1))
 (segment (start 141.9225 97.63125) (end 135.73125 91.44) (width 0.2) (layer "B.Cu") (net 1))
 (segment (start 135.73125 86.0575) (end 135.73125 68.94875) (width 0.2) (layer "B.Cu") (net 1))
 (segment (start 134.3025 97.63125) (end 135.66125 97.63125) (width 0.2) (layer "B.Cu") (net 5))
 (segment (start 135.66125 97.63125) (end 145.95 107.92) (width 0.2) (layer "B.Cu") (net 5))
 (segment (start 164.7825 97.63125) (end 164.7825 107.5625) (width 0.2) (layer "B.Cu") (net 9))
 (segment (start 164.7825 107.5625) (end 165.13 107.91) (width 0.2) (layer "B.Cu") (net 9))
 (segment (start 125.455 125.845) (end 126.72 127.11) (width 0.2) (layer "F.Cu") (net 4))
 (segment (start 116.68125 125.845) (end 125.455 125.845) (width 0.2) (layer "F.Cu") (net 4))
 (segment (start 158.63 127.12) (end 159.54375 126.20625) (width 0.2) (layer "F.Cu") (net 24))
 (segment (start 145.9 127.12) (end 158.63 127.12) (width 0.2) (layer "F.Cu") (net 24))
 (via (at 159.54375 126.20625) (size 0.6) (drill 0.3) (layers "F.Cu" "B.Cu") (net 24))
 (segment (start 161.925 126.20625) (end 183.35625 104.775) (width 0.2) (layer "B.Cu") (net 24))
 (segment (start 159.54375 126.20625) (end 161.925 126.20625) (width 0.2) (layer "B.Cu") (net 24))
 (segment (start 165.11 127.12) (end 182.08125 127.12) (width 0.2) (layer "F.Cu") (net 21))
 (segment (start 182.08125 127.12) (end 183.35625 125.845) (width 0.2) (layer "F.Cu") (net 21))
 (segment (start 180.60125 69.05625) (end 180.60125 79.63683) (width 0.2) (layer "F.Cu") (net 8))
 (segment (start 180.60125 79.63683) (end 183.4625 82.49808) (width 0.2) (layer "F.Cu") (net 8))
 (segment (start 129.9835 88.06275) (end 136.93725 88.06275) (width 0.2) (layer "F.Cu") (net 18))
 (segment (start 136.93725 88.06275) (end 157.17 67.83) (width 0.2) (layer "F.Cu") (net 18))
 (segment (start 127.65875 90.3875) (end 129.9835 88.06275) (width 0.2) (layer "F.Cu") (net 18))
 (segment (start 140.05625 72.91) (end 141.93 72.91) (width 0.2) (layer "F.Cu") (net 10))
 (segment (start 127.65875 85.3075) (end 140.05625 72.91) (width 0.2) (layer "F.Cu") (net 10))
 (segment (start 140.05625 75.45) (end 141.93 75.45) (width 0.2) (layer "F.Cu") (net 11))
 (segment (start 127.65875 87.8475) (end 140.05625 75.45) (width 0.2) (layer "F.Cu") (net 11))
 (segment (start 133.09125 105.38) (end 152.3 105.38) (width 0.2) (layer "F.Cu") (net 6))
 (segment (start 171.48 105.37) (end 152.31 105.37) (width 0.2) (layer "F.Cu") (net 6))
 (segment (start 152.31 105.37) (end 152.3 105.38) (width 0.2) (layer "F.Cu") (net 6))
 (segment (start 152.4 78.3) (end 141.93 67.83) (width 0.2) (layer "B.Cu") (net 6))
 (segment (start 152.4 78.3) (end 152.4 104.284214) (width 0.2) (layer "B.Cu") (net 6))
 (segment (start 152.4 104.284214) (end 152.801 104.685214) (width 0.2) (layer "B.Cu") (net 6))
 (segment (start 152.24 124.57) (end 152.25 124.58) (width 0.2) (layer "F.Cu") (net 7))
 (segment (start 133.07 124.57) (end 152.24 124.57) (width 0.2) (layer "F.Cu") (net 7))
 (segment (start 152.25 124.58) (end 171.46 124.58) (width 0.2) (layer "F.Cu") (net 7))
 (segment (start 150.999 103.450314) (end 150.999 79.439) (width 0.2) (layer "B.Cu") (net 7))
 (segment (start 152.4 124.1425) (end 152.4 104.851314) (width 0.2) (layer "B.Cu") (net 7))
 (segment (start 150.999 79.439) (end 141.93 70.37) (width 0.2) (layer "B.Cu") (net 7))
 (segment (start 152.4 104.851314) (end 150.999 103.450314) (width 0.2) (layer "B.Cu") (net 7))
 (segment (start 178.8125 87.49808) (end 164.22442 72.91) (width 0.2) (layer "B.Cu") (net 16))
 (segment (start 183.4625 87.49808) (end 178.8125 87.49808) (width 0.2) (layer "B.Cu") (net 16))
 (segment (start 164.22442 72.91) (end 158.27125 72.91) (width 0.2) (layer "B.Cu") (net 16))
 (segment (start 158.27125 72.91) (end 157.17 72.91) (width 0.2) (layer "B.Cu") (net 16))
 (segment (start 157.17 77.99) (end 157.17 81.65875) (width 0.2) (layer "B.Cu") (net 14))
 (segment (start 159.6575 78.19308) (end 168.9625 87.49808) (width 0.2) (layer "B.Cu") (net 14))
 (segment (start 168.9625 81.28933) (end 168.9625 82.49808) (width 0.2) (layer "B.Cu") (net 15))
 (segment (start 163.12317 75.45) (end 168.9625 81.28933) (width 0.2) (layer "B.Cu") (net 15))
 (segment (start 157.17 75.45) (end 163.12317 75.45) (width 0.2) (layer "B.Cu") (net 15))
 (segment (start 183.35625 112.395) (end 184.45725 113.496) (width 0.2) (layer "F.Cu") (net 3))
 (segment (start 116.68125 133.465) (end 183.35625 133.465) (width 0.2) (layer "F.Cu") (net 3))
 (segment (start 177.259407 103.804407) (end 180.101 100.962814) (width 0.2) (layer "F.Cu") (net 3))
 (segment (start 184.45725 132.364) (end 183.35625 133.465) (width 0.2) (layer "F.Cu") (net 3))
 (segment (start 172.98125 78.60525) (end 172.98125 69.05625) (width 0.2) (layer "F.Cu") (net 3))
 (segment (start 183.35625 109.90125) (end 183.35625 112.395) (width 0.2) (layer "F.Cu") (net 3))
 (segment (start 177.259407 103.804407) (end 183.35625 109.90125) (width 0.2) (layer "F.Cu") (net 3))
 (segment (start 180.101 100.962814) (end 180.101 85.725) (width 0.2) (layer "F.Cu") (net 3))
 (segment (start 184.45725 113.496) (end 184.45725 132.364) (width 0.2) (layer "F.Cu") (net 3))
 (segment (start 180.101 85.725) (end 172.98125 78.60525) (width 0.2) (layer "F.Cu") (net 3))
 (segment (start 167.38567 69.05625) (end 172.98125 69.05625) (width 0.2) (layer "B.Cu") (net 3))
 (segment (start 167.22242 68.893) (end 167.38567 69.05625) (width 0.2) (layer "B.Cu") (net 3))
 (segment (start 145.533 68.893) (end 167.22242 68.893) (width 0.2) (layer "B.Cu") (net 3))
 (segment (start 141.93 65.29) (end 145.533 68.893) (width 0.2) (layer "B.Cu") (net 3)))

